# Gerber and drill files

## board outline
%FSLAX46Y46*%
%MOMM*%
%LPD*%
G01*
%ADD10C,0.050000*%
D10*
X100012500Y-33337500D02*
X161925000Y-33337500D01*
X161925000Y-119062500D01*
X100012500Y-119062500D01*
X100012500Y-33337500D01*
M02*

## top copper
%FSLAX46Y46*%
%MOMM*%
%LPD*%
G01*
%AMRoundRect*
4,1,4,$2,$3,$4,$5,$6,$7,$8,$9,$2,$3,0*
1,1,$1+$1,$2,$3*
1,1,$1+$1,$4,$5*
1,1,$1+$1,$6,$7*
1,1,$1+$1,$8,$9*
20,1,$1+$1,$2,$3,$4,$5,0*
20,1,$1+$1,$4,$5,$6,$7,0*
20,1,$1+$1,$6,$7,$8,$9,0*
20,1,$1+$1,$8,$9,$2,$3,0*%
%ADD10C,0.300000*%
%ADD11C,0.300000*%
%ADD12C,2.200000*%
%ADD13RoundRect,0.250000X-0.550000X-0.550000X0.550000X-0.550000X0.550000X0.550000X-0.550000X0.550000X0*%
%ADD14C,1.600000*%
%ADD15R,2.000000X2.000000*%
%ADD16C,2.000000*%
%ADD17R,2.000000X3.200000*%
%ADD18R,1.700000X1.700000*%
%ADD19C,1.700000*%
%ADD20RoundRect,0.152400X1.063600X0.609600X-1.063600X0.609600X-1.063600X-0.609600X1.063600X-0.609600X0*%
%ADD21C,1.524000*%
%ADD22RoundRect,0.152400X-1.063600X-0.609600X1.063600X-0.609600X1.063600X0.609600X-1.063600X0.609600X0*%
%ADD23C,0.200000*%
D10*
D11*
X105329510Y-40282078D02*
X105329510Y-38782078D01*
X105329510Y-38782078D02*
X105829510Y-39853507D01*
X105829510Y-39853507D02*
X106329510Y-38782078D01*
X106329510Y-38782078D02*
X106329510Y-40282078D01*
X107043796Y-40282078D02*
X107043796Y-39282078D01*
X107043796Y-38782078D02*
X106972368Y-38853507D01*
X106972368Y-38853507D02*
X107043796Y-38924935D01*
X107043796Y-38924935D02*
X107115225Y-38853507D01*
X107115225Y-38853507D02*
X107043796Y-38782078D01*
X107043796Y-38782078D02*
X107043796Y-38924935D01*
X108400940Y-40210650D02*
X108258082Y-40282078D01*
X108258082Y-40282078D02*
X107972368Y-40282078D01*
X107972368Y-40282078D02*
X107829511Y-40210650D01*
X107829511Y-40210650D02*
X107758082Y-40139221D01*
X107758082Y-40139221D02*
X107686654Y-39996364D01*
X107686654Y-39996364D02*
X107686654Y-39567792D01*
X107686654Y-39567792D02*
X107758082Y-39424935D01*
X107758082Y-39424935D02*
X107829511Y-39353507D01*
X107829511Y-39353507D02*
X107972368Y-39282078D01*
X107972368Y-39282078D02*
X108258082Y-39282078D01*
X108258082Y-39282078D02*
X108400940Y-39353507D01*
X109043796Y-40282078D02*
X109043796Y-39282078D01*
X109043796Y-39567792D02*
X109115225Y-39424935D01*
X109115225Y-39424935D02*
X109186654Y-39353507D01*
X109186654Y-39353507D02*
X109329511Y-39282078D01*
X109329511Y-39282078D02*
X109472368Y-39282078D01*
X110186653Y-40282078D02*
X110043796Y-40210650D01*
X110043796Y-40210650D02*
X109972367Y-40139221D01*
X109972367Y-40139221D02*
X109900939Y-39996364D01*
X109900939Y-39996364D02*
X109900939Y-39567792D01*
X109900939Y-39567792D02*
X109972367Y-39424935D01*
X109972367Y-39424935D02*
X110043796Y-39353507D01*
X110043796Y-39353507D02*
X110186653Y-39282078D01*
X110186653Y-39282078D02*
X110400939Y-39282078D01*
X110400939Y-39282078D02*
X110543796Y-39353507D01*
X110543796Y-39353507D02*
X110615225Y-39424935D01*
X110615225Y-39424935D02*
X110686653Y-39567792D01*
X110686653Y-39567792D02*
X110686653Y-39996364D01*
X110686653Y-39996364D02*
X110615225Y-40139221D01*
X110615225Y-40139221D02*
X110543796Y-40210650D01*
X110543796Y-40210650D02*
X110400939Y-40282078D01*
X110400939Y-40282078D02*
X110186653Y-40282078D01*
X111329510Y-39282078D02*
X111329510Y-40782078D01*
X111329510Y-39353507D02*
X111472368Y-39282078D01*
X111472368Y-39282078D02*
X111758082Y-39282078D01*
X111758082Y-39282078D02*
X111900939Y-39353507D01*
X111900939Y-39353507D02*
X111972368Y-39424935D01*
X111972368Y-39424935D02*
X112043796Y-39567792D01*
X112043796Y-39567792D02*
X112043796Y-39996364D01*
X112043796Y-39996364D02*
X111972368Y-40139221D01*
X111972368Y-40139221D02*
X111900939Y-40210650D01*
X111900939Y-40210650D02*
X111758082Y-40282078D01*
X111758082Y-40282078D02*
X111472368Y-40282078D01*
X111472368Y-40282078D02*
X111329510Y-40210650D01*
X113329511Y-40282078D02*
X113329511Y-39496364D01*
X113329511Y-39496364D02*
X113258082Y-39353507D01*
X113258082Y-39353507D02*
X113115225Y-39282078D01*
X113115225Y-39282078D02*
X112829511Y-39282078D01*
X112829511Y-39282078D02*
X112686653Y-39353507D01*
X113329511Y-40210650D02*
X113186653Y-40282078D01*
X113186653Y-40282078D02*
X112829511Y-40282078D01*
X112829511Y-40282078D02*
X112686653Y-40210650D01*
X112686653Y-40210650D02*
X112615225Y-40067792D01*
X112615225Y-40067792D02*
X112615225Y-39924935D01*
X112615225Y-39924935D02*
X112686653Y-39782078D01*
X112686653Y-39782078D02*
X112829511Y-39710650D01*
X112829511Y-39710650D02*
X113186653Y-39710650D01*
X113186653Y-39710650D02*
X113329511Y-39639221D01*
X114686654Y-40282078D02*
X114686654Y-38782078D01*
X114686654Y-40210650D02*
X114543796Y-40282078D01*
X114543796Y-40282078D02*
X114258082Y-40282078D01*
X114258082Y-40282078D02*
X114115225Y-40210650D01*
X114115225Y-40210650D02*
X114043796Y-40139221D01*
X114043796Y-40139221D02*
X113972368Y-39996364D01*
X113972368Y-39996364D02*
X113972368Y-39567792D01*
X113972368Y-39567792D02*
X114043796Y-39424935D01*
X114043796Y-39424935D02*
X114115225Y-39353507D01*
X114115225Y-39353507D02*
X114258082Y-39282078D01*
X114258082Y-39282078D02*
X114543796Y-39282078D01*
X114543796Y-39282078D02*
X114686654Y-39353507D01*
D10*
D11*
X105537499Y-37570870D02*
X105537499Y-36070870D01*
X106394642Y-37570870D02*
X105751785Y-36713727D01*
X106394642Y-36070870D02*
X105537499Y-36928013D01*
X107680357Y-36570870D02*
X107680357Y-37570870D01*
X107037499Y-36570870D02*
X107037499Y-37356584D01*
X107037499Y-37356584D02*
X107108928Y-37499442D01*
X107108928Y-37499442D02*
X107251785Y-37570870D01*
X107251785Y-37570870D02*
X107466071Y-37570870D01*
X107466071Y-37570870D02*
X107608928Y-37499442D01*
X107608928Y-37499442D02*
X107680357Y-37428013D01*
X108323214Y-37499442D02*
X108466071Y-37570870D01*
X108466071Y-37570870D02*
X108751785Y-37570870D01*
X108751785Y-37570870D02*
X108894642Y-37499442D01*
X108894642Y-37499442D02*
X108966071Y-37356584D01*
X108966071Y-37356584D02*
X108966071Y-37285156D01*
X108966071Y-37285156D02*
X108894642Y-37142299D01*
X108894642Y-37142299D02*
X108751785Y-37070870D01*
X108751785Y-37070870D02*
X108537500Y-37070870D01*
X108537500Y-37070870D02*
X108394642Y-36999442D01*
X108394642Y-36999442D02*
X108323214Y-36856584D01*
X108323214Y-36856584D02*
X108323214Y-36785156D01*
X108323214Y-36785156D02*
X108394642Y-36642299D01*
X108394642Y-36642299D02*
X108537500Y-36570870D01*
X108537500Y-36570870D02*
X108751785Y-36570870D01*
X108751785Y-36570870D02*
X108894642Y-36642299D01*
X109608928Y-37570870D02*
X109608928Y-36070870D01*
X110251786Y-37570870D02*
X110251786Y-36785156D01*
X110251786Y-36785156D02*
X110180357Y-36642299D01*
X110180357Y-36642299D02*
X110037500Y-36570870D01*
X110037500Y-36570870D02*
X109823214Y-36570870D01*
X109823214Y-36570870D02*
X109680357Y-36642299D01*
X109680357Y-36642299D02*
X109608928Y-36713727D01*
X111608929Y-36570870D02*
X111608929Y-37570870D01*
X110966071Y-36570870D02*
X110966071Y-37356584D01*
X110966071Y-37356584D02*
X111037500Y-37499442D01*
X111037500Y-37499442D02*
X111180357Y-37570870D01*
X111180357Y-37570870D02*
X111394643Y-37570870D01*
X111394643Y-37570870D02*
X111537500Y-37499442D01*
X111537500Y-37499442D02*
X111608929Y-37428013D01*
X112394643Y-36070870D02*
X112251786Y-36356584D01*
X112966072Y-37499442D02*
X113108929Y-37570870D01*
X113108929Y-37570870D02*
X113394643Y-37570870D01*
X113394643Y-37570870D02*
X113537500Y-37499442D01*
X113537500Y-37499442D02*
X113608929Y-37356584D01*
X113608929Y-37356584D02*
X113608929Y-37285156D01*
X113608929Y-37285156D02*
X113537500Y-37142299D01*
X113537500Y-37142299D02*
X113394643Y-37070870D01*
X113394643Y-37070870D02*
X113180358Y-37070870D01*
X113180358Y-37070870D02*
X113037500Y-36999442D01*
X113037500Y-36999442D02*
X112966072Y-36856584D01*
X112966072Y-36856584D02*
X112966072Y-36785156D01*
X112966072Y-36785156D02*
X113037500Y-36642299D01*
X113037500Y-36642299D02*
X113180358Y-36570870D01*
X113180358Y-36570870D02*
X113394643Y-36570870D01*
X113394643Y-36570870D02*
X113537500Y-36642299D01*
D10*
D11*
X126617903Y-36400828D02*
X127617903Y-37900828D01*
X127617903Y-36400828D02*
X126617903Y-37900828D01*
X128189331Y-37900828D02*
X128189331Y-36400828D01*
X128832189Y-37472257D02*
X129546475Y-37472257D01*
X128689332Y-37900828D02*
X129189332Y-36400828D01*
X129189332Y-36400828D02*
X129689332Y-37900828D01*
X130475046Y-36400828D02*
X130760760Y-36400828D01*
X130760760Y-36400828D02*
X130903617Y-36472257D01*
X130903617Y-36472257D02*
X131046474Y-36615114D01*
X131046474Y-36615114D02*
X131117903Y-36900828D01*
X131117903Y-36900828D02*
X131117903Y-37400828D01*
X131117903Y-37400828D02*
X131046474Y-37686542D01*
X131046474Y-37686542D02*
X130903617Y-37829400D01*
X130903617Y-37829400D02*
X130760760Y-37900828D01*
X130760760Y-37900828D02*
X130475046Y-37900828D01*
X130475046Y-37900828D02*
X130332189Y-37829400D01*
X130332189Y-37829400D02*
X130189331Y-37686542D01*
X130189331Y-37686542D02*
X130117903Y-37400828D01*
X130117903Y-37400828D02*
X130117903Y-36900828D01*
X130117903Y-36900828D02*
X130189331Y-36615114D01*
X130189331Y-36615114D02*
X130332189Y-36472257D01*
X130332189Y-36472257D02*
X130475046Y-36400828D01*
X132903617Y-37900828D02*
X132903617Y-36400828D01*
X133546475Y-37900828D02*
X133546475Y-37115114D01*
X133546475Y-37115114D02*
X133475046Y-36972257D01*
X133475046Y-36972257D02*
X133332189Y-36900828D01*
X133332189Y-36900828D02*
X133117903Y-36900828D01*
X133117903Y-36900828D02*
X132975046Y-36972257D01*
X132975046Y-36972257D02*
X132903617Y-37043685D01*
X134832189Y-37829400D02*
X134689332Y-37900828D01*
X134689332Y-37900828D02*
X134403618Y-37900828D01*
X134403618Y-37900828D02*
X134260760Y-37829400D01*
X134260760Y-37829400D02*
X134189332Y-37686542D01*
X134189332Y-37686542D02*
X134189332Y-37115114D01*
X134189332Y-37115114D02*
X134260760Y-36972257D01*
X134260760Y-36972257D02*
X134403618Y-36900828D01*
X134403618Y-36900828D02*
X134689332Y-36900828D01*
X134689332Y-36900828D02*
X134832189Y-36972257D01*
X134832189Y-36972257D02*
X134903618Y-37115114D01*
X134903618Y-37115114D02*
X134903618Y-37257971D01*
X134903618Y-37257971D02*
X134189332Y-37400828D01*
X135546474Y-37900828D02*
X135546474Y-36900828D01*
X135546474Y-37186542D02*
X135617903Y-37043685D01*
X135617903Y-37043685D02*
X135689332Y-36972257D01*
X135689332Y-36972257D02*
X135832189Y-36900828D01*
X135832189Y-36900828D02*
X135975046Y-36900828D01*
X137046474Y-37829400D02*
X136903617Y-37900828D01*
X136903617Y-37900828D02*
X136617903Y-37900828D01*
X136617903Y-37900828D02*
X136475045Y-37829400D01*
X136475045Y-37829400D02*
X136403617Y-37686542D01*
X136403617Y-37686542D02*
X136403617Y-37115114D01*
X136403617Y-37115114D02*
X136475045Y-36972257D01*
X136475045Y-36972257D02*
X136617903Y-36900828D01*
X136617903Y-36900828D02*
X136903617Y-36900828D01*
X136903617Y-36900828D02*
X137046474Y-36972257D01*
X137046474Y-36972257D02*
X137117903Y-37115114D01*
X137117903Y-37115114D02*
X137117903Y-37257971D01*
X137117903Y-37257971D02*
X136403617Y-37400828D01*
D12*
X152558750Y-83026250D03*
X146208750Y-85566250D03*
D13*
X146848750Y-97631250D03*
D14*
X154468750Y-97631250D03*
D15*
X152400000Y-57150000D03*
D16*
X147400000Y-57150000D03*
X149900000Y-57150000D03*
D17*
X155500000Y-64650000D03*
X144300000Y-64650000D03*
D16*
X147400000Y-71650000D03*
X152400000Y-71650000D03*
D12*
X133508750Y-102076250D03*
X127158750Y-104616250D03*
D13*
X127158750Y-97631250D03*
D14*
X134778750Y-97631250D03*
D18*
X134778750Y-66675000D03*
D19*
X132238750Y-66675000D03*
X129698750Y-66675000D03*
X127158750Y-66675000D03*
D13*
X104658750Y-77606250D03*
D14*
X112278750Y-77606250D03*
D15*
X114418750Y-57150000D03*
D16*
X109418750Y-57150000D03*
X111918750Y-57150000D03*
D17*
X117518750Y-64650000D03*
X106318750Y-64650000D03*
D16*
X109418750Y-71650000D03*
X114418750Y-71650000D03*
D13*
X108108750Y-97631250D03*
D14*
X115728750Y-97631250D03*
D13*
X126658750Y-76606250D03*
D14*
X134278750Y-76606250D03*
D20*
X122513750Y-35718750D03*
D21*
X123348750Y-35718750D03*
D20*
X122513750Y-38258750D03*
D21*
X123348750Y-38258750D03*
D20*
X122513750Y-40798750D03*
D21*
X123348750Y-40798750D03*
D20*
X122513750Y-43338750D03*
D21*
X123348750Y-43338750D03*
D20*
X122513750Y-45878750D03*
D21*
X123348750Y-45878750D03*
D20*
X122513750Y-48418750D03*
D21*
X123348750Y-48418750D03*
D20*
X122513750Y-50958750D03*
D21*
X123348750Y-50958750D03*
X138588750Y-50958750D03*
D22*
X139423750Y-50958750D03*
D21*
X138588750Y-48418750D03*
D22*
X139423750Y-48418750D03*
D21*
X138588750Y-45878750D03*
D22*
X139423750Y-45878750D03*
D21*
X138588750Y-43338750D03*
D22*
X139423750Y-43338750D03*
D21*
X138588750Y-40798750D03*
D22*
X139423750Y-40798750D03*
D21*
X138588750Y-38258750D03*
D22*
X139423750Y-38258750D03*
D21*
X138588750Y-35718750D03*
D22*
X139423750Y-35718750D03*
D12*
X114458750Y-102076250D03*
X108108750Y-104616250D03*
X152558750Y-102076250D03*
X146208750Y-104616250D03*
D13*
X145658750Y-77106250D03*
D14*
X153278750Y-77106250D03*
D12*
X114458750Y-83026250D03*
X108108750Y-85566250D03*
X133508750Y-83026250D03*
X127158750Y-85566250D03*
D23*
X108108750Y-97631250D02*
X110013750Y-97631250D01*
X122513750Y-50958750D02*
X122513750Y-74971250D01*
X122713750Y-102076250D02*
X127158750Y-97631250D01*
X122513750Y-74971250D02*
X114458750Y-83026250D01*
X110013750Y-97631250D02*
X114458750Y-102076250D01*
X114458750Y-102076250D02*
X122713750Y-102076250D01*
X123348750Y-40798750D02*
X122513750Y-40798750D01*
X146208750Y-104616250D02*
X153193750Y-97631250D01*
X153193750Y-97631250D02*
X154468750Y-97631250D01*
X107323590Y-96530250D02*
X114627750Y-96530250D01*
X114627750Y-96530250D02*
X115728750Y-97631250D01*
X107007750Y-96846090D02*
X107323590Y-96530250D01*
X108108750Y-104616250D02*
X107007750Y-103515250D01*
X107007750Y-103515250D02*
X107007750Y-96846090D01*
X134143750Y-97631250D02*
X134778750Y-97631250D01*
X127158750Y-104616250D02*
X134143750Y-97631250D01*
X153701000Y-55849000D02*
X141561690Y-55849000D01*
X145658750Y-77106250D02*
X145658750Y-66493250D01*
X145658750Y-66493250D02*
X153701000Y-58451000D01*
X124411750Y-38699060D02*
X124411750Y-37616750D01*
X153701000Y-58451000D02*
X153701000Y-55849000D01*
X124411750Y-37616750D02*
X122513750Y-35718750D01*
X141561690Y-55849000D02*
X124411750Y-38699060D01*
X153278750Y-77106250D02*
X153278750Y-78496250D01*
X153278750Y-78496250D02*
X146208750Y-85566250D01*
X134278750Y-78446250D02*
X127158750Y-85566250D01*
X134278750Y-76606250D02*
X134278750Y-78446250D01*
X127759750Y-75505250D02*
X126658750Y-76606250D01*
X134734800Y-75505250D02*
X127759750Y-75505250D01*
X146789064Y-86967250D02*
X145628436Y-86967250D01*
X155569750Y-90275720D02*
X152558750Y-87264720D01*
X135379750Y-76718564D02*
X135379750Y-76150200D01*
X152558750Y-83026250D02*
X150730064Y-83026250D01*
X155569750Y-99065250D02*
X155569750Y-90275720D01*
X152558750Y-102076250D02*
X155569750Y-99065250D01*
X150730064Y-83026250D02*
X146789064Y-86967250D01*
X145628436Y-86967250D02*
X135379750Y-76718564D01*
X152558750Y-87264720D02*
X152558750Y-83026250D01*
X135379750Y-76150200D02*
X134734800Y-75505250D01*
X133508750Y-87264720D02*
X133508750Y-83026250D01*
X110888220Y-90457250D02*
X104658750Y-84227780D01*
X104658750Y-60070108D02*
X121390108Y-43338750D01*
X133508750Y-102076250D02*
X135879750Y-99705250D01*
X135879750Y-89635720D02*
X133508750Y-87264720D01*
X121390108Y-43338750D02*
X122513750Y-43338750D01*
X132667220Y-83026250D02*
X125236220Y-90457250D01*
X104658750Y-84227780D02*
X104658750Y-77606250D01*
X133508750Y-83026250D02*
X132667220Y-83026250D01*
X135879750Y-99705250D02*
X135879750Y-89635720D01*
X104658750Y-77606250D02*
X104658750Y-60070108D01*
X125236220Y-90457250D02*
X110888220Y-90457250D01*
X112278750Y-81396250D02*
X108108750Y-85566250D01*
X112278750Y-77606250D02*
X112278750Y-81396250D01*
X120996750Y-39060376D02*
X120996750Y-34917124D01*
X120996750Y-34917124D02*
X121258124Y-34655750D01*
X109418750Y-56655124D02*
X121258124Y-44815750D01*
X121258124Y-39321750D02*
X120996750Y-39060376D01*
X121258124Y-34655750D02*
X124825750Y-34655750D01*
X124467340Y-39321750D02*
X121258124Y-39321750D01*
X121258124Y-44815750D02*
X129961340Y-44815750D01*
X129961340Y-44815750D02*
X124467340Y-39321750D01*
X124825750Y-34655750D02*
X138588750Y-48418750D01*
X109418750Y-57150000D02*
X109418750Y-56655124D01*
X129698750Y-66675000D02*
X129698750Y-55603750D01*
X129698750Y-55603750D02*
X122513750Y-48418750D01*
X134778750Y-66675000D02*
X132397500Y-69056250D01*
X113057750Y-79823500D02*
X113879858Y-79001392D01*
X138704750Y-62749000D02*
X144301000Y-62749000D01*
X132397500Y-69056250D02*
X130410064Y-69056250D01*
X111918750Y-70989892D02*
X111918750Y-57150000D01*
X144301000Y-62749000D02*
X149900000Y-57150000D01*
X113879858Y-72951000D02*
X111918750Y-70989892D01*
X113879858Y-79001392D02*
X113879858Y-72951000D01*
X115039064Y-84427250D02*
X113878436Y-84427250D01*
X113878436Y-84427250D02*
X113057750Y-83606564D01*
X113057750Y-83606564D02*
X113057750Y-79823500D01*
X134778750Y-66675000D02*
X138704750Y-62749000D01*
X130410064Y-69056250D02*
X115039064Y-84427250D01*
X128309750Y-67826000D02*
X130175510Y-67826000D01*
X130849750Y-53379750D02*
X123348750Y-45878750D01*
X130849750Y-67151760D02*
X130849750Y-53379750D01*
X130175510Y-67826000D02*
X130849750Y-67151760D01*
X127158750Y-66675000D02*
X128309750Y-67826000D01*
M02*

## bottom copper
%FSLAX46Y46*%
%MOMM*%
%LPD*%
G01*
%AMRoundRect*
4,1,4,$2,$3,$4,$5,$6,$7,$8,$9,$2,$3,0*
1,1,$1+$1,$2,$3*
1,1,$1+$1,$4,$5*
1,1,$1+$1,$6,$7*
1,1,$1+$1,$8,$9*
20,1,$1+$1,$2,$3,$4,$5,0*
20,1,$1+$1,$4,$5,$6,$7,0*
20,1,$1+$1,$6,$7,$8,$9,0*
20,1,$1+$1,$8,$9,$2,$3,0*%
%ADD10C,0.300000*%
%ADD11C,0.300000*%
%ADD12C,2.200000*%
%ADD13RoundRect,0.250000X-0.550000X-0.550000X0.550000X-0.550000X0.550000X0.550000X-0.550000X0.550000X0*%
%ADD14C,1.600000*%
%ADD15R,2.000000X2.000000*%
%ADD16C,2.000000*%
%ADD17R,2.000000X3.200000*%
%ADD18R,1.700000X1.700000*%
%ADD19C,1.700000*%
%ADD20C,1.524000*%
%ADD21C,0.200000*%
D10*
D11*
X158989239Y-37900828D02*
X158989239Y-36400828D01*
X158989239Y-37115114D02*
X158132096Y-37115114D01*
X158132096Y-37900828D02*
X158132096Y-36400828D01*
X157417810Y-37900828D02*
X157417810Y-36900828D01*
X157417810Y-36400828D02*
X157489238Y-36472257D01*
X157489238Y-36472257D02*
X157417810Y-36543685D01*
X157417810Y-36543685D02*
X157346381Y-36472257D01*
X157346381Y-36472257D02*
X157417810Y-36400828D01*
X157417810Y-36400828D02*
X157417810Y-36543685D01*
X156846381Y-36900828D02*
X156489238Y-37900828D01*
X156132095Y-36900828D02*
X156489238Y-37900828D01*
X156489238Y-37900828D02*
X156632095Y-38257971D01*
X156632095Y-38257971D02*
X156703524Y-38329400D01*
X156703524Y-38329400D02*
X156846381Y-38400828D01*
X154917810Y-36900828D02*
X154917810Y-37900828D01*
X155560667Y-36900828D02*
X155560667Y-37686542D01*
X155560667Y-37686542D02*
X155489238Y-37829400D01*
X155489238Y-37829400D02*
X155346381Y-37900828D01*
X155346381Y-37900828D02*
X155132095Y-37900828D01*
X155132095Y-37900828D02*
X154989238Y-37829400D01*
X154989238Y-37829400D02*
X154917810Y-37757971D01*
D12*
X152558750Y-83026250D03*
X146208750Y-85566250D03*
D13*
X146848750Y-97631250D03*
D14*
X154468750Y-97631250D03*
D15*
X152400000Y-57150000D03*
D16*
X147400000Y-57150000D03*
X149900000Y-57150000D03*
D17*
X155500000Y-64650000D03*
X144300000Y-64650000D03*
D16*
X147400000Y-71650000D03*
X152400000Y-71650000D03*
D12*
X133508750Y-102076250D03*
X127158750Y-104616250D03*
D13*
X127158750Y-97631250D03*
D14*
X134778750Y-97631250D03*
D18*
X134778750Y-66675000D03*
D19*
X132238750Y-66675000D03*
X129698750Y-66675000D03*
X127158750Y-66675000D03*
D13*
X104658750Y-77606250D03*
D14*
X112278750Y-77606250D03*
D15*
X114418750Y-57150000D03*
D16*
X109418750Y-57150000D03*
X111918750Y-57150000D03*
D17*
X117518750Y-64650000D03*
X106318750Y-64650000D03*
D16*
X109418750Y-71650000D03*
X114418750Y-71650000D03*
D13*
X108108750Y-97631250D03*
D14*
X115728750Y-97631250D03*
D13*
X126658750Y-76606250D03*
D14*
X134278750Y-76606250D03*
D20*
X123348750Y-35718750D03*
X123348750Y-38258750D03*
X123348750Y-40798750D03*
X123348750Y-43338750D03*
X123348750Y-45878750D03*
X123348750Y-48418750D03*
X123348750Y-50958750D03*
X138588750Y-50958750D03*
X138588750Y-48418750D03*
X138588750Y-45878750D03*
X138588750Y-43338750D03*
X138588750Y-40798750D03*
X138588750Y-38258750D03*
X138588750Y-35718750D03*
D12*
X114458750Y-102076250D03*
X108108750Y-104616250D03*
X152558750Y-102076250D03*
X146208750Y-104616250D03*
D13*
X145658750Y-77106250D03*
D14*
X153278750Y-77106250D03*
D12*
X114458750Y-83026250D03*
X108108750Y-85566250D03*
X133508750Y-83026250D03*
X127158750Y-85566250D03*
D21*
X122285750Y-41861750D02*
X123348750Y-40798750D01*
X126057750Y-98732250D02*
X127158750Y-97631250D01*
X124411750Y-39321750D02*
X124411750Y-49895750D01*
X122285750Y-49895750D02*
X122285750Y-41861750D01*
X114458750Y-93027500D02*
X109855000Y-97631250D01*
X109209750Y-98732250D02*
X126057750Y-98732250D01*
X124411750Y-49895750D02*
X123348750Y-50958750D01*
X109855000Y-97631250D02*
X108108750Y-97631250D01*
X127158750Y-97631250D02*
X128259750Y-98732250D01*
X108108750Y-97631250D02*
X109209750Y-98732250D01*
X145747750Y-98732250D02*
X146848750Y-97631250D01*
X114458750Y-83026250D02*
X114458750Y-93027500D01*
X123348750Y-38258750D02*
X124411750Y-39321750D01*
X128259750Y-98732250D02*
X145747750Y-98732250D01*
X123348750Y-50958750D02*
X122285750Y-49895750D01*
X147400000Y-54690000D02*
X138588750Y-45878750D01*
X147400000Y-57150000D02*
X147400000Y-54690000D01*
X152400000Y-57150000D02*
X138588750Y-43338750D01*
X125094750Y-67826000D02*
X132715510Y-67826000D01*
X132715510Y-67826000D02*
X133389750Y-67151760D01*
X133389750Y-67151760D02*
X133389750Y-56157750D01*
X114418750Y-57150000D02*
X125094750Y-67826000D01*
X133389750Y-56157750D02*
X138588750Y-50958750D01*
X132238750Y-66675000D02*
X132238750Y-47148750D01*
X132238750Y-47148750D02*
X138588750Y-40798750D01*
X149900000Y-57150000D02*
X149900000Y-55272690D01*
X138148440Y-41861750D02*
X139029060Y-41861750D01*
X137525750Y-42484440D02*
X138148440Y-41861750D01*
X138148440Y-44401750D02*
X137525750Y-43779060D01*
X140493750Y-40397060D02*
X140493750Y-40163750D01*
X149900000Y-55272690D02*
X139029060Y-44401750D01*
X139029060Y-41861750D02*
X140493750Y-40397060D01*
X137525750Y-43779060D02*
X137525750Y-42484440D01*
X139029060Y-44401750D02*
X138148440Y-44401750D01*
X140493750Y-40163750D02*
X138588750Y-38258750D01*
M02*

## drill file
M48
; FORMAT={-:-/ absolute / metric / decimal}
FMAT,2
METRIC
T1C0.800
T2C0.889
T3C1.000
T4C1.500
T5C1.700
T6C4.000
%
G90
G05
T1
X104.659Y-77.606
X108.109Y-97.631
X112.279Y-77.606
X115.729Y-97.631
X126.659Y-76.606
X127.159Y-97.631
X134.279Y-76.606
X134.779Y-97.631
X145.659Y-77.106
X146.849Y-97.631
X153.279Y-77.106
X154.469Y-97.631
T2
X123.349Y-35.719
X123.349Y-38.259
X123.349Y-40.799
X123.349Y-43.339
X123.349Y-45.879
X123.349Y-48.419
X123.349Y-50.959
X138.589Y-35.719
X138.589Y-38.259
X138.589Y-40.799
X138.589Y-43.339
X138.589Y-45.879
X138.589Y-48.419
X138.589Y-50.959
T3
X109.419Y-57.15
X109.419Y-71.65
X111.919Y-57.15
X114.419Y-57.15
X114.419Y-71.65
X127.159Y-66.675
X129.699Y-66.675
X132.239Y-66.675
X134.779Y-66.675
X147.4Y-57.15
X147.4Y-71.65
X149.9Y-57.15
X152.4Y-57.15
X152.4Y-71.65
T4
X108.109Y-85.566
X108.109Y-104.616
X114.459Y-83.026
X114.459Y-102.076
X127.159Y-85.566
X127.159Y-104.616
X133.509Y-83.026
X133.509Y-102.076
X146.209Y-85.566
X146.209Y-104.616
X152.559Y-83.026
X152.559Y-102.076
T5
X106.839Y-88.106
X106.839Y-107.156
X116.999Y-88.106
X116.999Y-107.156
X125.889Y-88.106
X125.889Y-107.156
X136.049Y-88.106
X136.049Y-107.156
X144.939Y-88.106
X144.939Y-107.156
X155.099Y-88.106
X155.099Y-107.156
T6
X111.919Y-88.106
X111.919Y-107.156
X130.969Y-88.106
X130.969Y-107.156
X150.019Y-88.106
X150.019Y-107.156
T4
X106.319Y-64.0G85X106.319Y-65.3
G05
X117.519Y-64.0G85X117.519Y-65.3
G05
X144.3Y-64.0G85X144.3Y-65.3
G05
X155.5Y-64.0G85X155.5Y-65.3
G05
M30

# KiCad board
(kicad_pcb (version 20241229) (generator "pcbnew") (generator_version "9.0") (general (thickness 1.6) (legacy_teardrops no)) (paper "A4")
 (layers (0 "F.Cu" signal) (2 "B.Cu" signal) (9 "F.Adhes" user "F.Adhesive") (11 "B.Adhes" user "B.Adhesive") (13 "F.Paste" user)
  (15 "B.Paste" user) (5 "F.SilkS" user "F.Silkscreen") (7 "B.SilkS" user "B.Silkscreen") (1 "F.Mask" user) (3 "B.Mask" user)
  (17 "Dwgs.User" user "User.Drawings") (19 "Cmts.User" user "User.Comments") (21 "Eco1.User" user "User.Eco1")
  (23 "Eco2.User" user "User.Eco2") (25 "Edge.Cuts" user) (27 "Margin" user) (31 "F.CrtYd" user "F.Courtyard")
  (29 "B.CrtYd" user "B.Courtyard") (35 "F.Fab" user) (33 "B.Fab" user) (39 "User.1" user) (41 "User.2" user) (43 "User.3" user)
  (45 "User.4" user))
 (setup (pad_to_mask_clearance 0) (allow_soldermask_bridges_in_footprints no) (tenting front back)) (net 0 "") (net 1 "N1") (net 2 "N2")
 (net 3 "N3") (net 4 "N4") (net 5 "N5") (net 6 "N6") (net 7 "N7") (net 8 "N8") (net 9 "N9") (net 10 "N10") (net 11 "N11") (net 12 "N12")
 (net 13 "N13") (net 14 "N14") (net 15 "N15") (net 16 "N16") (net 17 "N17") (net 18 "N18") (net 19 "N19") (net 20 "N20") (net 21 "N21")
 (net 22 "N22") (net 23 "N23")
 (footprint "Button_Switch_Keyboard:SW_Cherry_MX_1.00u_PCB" (layer "F.Cu") (at 152.55875 83.02625)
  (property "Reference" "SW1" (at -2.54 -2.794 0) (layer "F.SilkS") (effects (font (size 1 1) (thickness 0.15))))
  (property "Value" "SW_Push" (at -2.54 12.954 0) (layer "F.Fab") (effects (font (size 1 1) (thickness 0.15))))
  (pad "" np_thru_hole circle (at -7.62 5.08) (size 1.7 1.7) (drill 1.7) (layers "*.Cu" "*.Mask"))
  (pad "" np_thru_hole circle (at -2.54 5.08) (size 4 4) (drill 4) (layers "*.Cu" "*.Mask"))
  (pad "" np_thru_hole circle (at 2.54 5.08) (size 1.7 1.7) (drill 1.7) (layers "*.Cu" "*.Mask"))
  (pad "1" thru_hole circle (at 0 0) (size 2.2 2.2) (drill 1.5) (layers "*.Cu" "*.Mask") (remove_unused_layers no) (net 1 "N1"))
  (pad "2" thru_hole circle (at -6.35 2.54) (size 2.2 2.2) (drill 1.5) (layers "*.Cu" "*.Mask") (remove_unused_layers no) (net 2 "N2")))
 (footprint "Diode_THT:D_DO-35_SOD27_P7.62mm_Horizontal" (layer "F.Cu") (at 146.84875 97.63125)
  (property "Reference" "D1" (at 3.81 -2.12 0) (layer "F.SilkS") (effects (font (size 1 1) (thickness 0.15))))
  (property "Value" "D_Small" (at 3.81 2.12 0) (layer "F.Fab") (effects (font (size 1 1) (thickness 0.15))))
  (pad "1" thru_hole roundrect (at 0 0) (size 1.6 1.6) (drill 0.8) (layers "*.Cu" "*.Mask") (remove_unused_layers no)
   (roundrect_rratio 0.15625) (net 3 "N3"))
  (pad "2" thru_hole circle (at 7.62 0) (size 1.6 1.6) (drill 0.8) (layers "*.Cu" "*.Mask") (remove_unused_layers no) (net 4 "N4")))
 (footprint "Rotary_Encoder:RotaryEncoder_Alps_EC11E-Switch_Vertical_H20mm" (layer "F.Cu") (at 152.4 57.15 -90)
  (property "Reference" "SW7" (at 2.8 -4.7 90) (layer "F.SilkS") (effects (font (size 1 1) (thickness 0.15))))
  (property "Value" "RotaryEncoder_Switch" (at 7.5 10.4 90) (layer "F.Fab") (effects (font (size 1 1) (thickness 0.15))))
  (pad "A" thru_hole rect (at 0 0 270) (size 2 2) (drill 1) (layers "*.Cu" "*.Mask") (remove_unused_layers no) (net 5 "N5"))
  (pad "B" thru_hole circle (at 0 5 270) (size 2 2) (drill 1) (layers "*.Cu" "*.Mask") (remove_unused_layers no) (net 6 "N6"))
  (pad "C" thru_hole circle (at 0 2.5 270) (size 2 2) (drill 1) (layers "*.Cu" "*.Mask") (remove_unused_layers no) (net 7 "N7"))
  (pad "MP" thru_hole rect (at 7.5 -3.1 270) (size 3.2 2) (drill oval 2.8 1.5) (layers "*.Cu" "*.Mask") (remove_unused_layers no))
  (pad "MP" thru_hole rect (at 7.5 8.1 270) (size 3.2 2) (drill oval 2.8 1.5) (layers "*.Cu" "*.Mask") (remove_unused_layers no))
  (pad "S1" thru_hole circle (at 14.5 5 270) (size 2 2) (drill 1) (layers "*.Cu" "*.Mask") (remove_unused_layers no) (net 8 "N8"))
  (pad "S2" thru_hole circle (at 14.5 0 270) (size 2 2) (drill 1) (layers "*.Cu" "*.Mask") (remove_unused_layers no) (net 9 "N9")))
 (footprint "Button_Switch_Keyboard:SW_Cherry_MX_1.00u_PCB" (layer "F.Cu") (at 133.50875 102.07625)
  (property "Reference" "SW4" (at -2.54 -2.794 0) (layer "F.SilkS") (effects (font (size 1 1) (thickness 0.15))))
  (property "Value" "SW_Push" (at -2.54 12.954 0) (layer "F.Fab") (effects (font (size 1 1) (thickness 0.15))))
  (pad "" np_thru_hole circle (at -7.62 5.08) (size 1.7 1.7) (drill 1.7) (layers "*.Cu" "*.Mask"))
  (pad "" np_thru_hole circle (at -2.54 5.08) (size 4 4) (drill 4) (layers "*.Cu" "*.Mask"))
  (pad "" np_thru_hole circle (at 2.54 5.08) (size 1.7 1.7) (drill 1.7) (layers "*.Cu" "*.Mask"))
  (pad "1" thru_hole circle (at 0 0) (size 2.2 2.2) (drill 1.5) (layers "*.Cu" "*.Mask") (remove_unused_layers no) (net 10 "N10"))
  (pad "2" thru_hole circle (at -6.35 2.54) (size 2.2 2.2) (drill 1.5) (layers "*.Cu" "*.Mask") (remove_unused_layers no) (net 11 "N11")))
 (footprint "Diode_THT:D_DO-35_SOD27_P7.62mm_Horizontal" (layer "F.Cu") (at 127.15875 97.63125)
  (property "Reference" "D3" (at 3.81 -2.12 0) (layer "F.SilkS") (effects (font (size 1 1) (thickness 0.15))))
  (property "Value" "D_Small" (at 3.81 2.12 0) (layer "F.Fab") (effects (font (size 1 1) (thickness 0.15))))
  (pad "1" thru_hole roundrect (at 0 0) (size 1.6 1.6) (drill 0.8) (layers "*.Cu" "*.Mask") (remove_unused_layers no)
   (roundrect_rratio 0.15625) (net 3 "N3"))
  (pad "2" thru_hole circle (at 7.62 0) (size 1.6 1.6) (drill 0.8) (layers "*.Cu" "*.Mask") (remove_unused_layers no) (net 11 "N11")))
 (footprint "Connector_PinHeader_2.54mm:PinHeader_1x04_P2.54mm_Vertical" (layer "F.Cu") (at 134.77875 66.675 -90)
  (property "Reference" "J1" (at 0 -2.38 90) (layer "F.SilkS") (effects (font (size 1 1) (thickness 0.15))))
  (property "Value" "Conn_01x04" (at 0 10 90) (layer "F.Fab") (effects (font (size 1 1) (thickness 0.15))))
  (pad "1" thru_hole rect (at 0 0 270) (size 1.7 1.7) (drill 1) (layers "*.Cu" "*.Mask") (remove_unused_layers no) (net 7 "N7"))
  (pad "2" thru_hole circle (at 0 2.54 270) (size 1.7 1.7) (drill 1) (layers "*.Cu" "*.Mask") (remove_unused_layers no) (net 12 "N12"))
  (pad "3" thru_hole circle (at 0 5.08 270) (size 1.7 1.7) (drill 1) (layers "*.Cu" "*.Mask") (remove_unused_layers no) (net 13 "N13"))
  (pad "4" thru_hole circle (at 0 7.62 270) (size 1.7 1.7) (drill 1) (layers "*.Cu" "*.Mask") (remove_unused_layers no) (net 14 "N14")))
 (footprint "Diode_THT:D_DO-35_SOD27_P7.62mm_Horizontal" (layer "F.Cu") (at 104.65875 77.60625)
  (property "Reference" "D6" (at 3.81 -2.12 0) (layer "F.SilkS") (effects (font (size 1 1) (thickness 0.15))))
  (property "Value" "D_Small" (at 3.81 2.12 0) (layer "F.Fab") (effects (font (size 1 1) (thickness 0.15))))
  (pad "1" thru_hole roundrect (at 0 0) (size 1.6 1.6) (drill 0.8) (layers "*.Cu" "*.Mask") (remove_unused_layers no)
   (roundrect_rratio 0.15625) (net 10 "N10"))
  (pad "2" thru_hole circle (at 7.62 0) (size 1.6 1.6) (drill 0.8) (layers "*.Cu" "*.Mask") (remove_unused_layers no) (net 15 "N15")))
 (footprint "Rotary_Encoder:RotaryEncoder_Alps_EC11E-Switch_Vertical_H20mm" (layer "F.Cu") (at 114.41875 57.15 -90)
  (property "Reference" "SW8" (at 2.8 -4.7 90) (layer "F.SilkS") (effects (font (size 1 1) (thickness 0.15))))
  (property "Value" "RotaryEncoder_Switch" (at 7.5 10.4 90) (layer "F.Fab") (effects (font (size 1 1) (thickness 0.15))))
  (pad "A" thru_hole rect (at 0 0 270) (size 2 2) (drill 1) (layers "*.Cu" "*.Mask") (remove_unused_layers no) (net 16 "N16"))
  (pad "B" thru_hole circle (at 0 5 270) (size 2 2) (drill 1) (layers "*.Cu" "*.Mask") (remove_unused_layers no) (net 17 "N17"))
  (pad "C" thru_hole circle (at 0 2.5 270) (size 2 2) (drill 1) (layers "*.Cu" "*.Mask") (remove_unused_layers no) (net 7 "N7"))
  (pad "MP" thru_hole rect (at 7.5 -3.1 270) (size 3.2 2) (drill oval 2.8 1.5) (layers "*.Cu" "*.Mask") (remove_unused_layers no))
  (pad "MP" thru_hole rect (at 7.5 8.1 270) (size 3.2 2) (drill oval 2.8 1.5) (layers "*.Cu" "*.Mask") (remove_unused_layers no))
  (pad "S1" thru_hole circle (at 14.5 5 270) (size 2 2) (drill 1) (layers "*.Cu" "*.Mask") (remove_unused_layers no) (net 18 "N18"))
  (pad "S2" thru_hole circle (at 14.5 0 270) (size 2 2) (drill 1) (layers "*.Cu" "*.Mask") (remove_unused_layers no) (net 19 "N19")))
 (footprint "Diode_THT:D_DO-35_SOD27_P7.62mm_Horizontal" (layer "F.Cu") (at 108.10875 97.63125)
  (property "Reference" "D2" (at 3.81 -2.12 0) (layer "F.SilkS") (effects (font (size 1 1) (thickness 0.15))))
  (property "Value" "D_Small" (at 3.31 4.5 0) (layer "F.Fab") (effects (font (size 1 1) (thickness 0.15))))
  (pad "1" thru_hole roundrect (at 0 0) (size 1.6 1.6) (drill 0.8) (layers "*.Cu" "*.Mask") (remove_unused_layers no)
   (roundrect_rratio 0.15625) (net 3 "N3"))
  (pad "2" thru_hole circle (at 7.62 0) (size 1.6 1.6) (drill 0.8) (layers "*.Cu" "*.Mask") (remove_unused_layers no) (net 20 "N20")))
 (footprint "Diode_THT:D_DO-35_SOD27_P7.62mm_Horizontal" (layer "F.Cu") (at 126.65875 76.60625)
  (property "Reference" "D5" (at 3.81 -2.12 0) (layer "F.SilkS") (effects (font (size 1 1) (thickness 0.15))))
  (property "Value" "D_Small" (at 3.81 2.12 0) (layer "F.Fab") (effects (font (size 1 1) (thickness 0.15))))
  (pad "1" thru_hole roundrect (at 0 0) (size 1.6 1.6) (drill 0.8) (layers "*.Cu" "*.Mask") (remove_unused_layers no)
   (roundrect_rratio 0.15625) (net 1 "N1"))
  (pad "2" thru_hole circle (at 7.62 0) (size 1.6 1.6) (drill 0.8) (layers "*.Cu" "*.Mask") (remove_unused_layers no) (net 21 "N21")))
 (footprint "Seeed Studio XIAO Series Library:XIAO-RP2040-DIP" (layer "F.Cu") (at 130.96875 43.33875)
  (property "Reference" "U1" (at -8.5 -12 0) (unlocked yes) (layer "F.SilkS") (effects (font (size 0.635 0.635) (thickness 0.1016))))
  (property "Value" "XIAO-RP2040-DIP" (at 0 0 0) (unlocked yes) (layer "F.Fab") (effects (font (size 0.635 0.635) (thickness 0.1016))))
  (pad "1" smd roundrect (at -8.455 -7.62 180) (size 2.432 1.524) (layers "F.Cu" "F.Mask") (roundrect_rratio 0.1) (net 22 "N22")
   (thermal_bridge_angle 45))
  (pad "1" thru_hole circle (at -7.62 -7.62 180) (size 1.524 1.524) (drill 0.889) (layers "*.Cu" "*.Mask") (remove_unused_layers no)
   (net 22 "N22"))
  (pad "2" smd roundrect (at -8.455 -5.08 180) (size 2.432 1.524) (layers "F.Cu" "F.Mask") (roundrect_rratio 0.1) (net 3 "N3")
   (thermal_bridge_angle 45))
  (pad "2" thru_hole circle (at -7.62 -5.08 180) (size 1.524 1.524) (drill 0.889) (layers "*.Cu" "*.Mask") (remove_unused_layers no)
   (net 3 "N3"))
  (pad "3" smd roundrect (at -8.455 -2.54 180) (size 2.432 1.524) (layers "F.Cu" "F.Mask") (roundrect_rratio 0.1) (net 3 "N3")
   (thermal_bridge_angle 45))
  (pad "3" thru_hole circle (at -7.62 -2.54 180) (size 1.524 1.524) (drill 0.889) (layers "*.Cu" "*.Mask") (remove_unused_layers no)
   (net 3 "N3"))
  (pad "4" smd roundrect (at -8.455 0 180) (size 2.432 1.524) (layers "F.Cu" "F.Mask") (roundrect_rratio 0.1) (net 10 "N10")
   (thermal_bridge_angle 45))
  (pad "4" thru_hole circle (at -7.62 0 180) (size 1.524 1.524) (drill 0.889) (layers "*.Cu" "*.Mask") (remove_unused_layers no)
   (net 10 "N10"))
  (pad "5" smd roundrect (at -8.455 2.54 180) (size 2.432 1.524) (layers "F.Cu" "F.Mask") (roundrect_rratio 0.1) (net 14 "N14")
   (thermal_bridge_angle 45))
  (pad "5" thru_hole circle (at -7.62 2.54 180) (size 1.524 1.524) (drill 0.889) (layers "*.Cu" "*.Mask") (remove_unused_layers no)
   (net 14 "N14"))
  (pad "6" smd roundrect (at -8.455 5.08 180) (size 2.432 1.524) (layers "F.Cu" "F.Mask") (roundrect_rratio 0.1) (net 13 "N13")
   (thermal_bridge_angle 45))
  (pad "6" thru_hole circle (at -7.62 5.08 180) (size 1.524 1.524) (drill 0.889) (layers "*.Cu" "*.Mask") (remove_unused_layers no)
   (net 13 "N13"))
  (pad "7" smd roundrect (at -8.455 7.62 180) (size 2.432 1.524) (layers "F.Cu" "F.Mask") (roundrect_rratio 0.1) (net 3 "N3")
   (thermal_bridge_angle 45))
  (pad "7" thru_hole circle (at -7.62 7.62 180) (size 1.524 1.524) (drill 0.889) (layers "*.Cu" "*.Mask") (remove_unused_layers no)
   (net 3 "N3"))
  (pad "8" thru_hole circle (at 7.62 7.62) (size 1.524 1.524) (drill 0.889) (layers "*.Cu" "*.Mask") (remove_unused_layers no)
   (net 16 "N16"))
  (pad "8" smd roundrect (at 8.455 7.62) (size 2.432 1.524) (layers "F.Cu" "F.Mask") (roundrect_rratio 0.1) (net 16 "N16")
   (thermal_bridge_angle 45))
  (pad "9" thru_hole circle (at 7.62 5.08) (size 1.524 1.524) (drill 0.889) (layers "*.Cu" "*.Mask") (remove_unused_layers no)
   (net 17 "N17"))
  (pad "9" smd roundrect (at 8.455 5.08) (size 2.432 1.524) (layers "F.Cu" "F.Mask") (roundrect_rratio 0.1) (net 17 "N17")
   (thermal_bridge_angle 45))
  (pad "10" thru_hole circle (at 7.62 2.54) (size 1.524 1.524) (drill 0.889) (layers "*.Cu" "*.Mask") (remove_unused_layers no) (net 6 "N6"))
  (pad "10" smd roundrect (at 8.455 2.54) (size 2.432 1.524) (layers "F.Cu" "F.Mask") (roundrect_rratio 0.1) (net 6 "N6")
   (thermal_bridge_angle 45))
  (pad "11" thru_hole circle (at 7.62 0) (size 1.524 1.524) (drill 0.889) (layers "*.Cu" "*.Mask") (remove_unused_layers no) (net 5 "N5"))
  (pad "11" smd roundrect (at 8.455 0) (size 2.432 1.524) (layers "F.Cu" "F.Mask") (roundrect_rratio 0.1) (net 5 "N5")
   (thermal_bridge_angle 45))
  (pad "12" thru_hole circle (at 7.62 -2.54) (size 1.524 1.524) (drill 0.889) (layers "*.Cu" "*.Mask") (remove_unused_layers no)
   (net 12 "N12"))
  (pad "12" smd roundrect (at 8.455 -2.54) (size 2.432 1.524) (layers "F.Cu" "F.Mask") (roundrect_rratio 0.1) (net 12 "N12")
   (thermal_bridge_angle 45))
  (pad "13" thru_hole circle (at 7.62 -5.08) (size 1.524 1.524) (drill 0.889) (layers "*.Cu" "*.Mask") (remove_unused_layers no)
   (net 7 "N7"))
  (pad "13" smd roundrect (at 8.455 -5.08) (size 2.432 1.524) (layers "F.Cu" "F.Mask") (roundrect_rratio 0.1) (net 7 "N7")
   (thermal_bridge_angle 45))
  (pad "14" thru_hole circle (at 7.62 -7.62) (size 1.524 1.524) (drill 0.889) (layers "*.Cu" "*.Mask") (remove_unused_layers no)
   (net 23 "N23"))
  (pad "14" smd roundrect (at 8.455 -7.62) (size 2.432 1.524) (layers "F.Cu" "F.Mask") (roundrect_rratio 0.1) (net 23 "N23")
   (thermal_bridge_angle 45)))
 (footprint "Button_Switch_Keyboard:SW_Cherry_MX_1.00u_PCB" (layer "F.Cu") (at 114.45875 102.07625)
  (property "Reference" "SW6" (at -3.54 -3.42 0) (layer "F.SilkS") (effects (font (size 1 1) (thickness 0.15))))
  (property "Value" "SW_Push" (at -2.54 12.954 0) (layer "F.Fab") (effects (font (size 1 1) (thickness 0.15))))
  (pad "" np_thru_hole circle (at -7.62 5.08) (size 1.7 1.7) (drill 1.7) (layers "*.Cu" "*.Mask"))
  (pad "" np_thru_hole circle (at -2.54 5.08) (size 4 4) (drill 4) (layers "*.Cu" "*.Mask"))
  (pad "" np_thru_hole circle (at 2.54 5.08) (size 1.7 1.7) (drill 1.7) (layers "*.Cu" "*.Mask"))
  (pad "1" thru_hole circle (at 0 0) (size 2.2 2.2) (drill 1.5) (layers "*.Cu" "*.Mask") (remove_unused_layers no) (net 3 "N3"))
  (pad "2" thru_hole circle (at -6.35 2.54) (size 2.2 2.2) (drill 1.5) (layers "*.Cu" "*.Mask") (remove_unused_layers no) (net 20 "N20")))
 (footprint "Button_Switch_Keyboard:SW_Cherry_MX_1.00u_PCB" (layer "F.Cu") (at 152.55875 102.07625)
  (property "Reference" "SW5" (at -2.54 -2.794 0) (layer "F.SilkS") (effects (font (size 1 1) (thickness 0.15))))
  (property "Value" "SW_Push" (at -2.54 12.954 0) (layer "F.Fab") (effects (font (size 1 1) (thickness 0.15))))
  (pad "" np_thru_hole circle (at -7.62 5.08) (size 1.7 1.7) (drill 1.7) (layers "*.Cu" "*.Mask"))
  (pad "" np_thru_hole circle (at -2.54 5.08) (size 4 4) (drill 4) (layers "*.Cu" "*.Mask"))
  (pad "" np_thru_hole circle (at 2.54 5.08) (size 1.7 1.7) (drill 1.7) (layers "*.Cu" "*.Mask"))
  (pad "1" thru_hole circle (at 0 0) (size 2.2 2.2) (drill 1.5) (layers "*.Cu" "*.Mask") (remove_unused_layers no) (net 1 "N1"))
  (pad "2" thru_hole circle (at -6.35 2.54) (size 2.2 2.2) (drill 1.5) (layers "*.Cu" "*.Mask") (remove_unused_layers no) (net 4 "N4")))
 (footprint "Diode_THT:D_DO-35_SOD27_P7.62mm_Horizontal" (layer "F.Cu") (at 145.65875 77.10625)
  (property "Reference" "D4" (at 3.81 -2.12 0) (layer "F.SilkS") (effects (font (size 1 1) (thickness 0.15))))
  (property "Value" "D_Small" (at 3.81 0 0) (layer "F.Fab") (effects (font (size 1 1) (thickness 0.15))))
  (pad "1" thru_hole roundrect (at 0 0) (size 1.6 1.6) (drill 0.8) (layers "*.Cu" "*.Mask") (remove_unused_layers no)
   (roundrect_rratio 0.15625) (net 22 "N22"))
  (pad "2" thru_hole circle (at 7.62 0) (size 1.6 1.6) (drill 0.8) (layers "*.Cu" "*.Mask") (remove_unused_layers no) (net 2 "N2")))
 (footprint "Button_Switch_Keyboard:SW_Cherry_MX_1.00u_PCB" (layer "F.Cu") (at 114.45875 83.02625)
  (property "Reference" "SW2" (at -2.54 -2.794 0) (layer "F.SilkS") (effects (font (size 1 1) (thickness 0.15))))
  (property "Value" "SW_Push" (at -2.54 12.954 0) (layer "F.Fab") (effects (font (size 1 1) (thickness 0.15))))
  (pad "" np_thru_hole circle (at -7.62 5.08) (size 1.7 1.7) (drill 1.7) (layers "*.Cu" "*.Mask"))
  (pad "" np_thru_hole circle (at -2.54 5.08) (size 4 4) (drill 4) (layers "*.Cu" "*.Mask"))
  (pad "" np_thru_hole circle (at 2.54 5.08) (size 1.7 1.7) (drill 1.7) (layers "*.Cu" "*.Mask"))
  (pad "1" thru_hole circle (at 0 0) (size 2.2 2.2) (drill 1.5) (layers "*.Cu" "*.Mask") (remove_unused_layers no) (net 3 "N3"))
  (pad "2" thru_hole circle (at -6.35 2.54) (size 2.2 2.2) (drill 1.5) (layers "*.Cu" "*.Mask") (remove_unused_layers no) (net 15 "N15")))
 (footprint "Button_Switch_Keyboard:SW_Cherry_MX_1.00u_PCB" (layer "F.Cu") (at 133.50875 83.02625)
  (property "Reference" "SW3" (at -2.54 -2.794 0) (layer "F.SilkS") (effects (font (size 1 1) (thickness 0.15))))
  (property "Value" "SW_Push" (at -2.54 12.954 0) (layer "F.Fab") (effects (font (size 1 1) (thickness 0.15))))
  (pad "" np_thru_hole circle (at -7.62 5.08) (size 1.7 1.7) (drill 1.7) (layers "*.Cu" "*.Mask"))
  (pad "" np_thru_hole circle (at -2.54 5.08) (size 4 4) (drill 4) (layers "*.Cu" "*.Mask"))
  (pad "" np_thru_hole circle (at 2.54 5.08) (size 1.7 1.7) (drill 1.7) (layers "*.Cu" "*.Mask"))
  (pad "1" thru_hole circle (at 0 0) (size 2.2 2.2) (drill 1.5) (layers "*.Cu" "*.Mask") (remove_unused_layers no) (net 10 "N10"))
  (pad "2" thru_hole circle (at -6.35 2.54) (size 2.2 2.2) (drill 1.5) (layers "*.Cu" "*.Mask") (remove_unused_layers no) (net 21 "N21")))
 (gr_rect (start 100.0125 33.3375) (end 161.925 119.0625) (stroke (width 0.05) (type default)) (fill no) (layer "Edge.Cuts"))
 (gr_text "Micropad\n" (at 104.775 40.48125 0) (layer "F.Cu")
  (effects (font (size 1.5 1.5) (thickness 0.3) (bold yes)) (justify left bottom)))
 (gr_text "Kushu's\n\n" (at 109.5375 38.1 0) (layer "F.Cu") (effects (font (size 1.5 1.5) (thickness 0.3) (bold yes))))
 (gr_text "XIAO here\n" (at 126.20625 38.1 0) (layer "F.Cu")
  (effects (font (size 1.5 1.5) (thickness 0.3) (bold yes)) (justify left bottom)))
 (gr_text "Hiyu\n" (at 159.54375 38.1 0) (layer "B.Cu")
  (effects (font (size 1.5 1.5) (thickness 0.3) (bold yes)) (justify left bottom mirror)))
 (segment (start 108.10875 97.63125) (end 110.01375 97.63125) (width 0.2) (layer "F.Cu") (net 3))
 (segment (start 122.51375 50.95875) (end 122.51375 74.97125) (width 0.2) (layer "F.Cu") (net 3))
 (segment (start 122.71375 102.07625) (end 127.15875 97.63125) (width 0.2) (layer "F.Cu") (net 3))
 (segment (start 122.51375 74.97125) (end 114.45875 83.02625) (width 0.2) (layer "F.Cu") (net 3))
 (segment (start 110.01375 97.63125) (end 114.45875 102.07625) (width 0.2) (layer "F.Cu") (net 3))
 (segment (start 114.45875 102.07625) (end 122.71375 102.07625) (width 0.2) (layer "F.Cu") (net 3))
 (segment (start 123.34875 40.79875) (end 122.51375 40.79875) (width 0.2) (layer "F.Cu") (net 3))
 (segment (start 122.28575 41.86175) (end 123.34875 40.79875) (width 0.2) (layer "B.Cu") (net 3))
 (segment (start 126.05775 98.73225) (end 127.15875 97.63125) (width 0.2) (layer "B.Cu") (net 3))
 (segment (start 124.41175 39.32175) (end 124.41175 49.89575) (width 0.2) (layer "B.Cu") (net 3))
 (segment (start 122.28575 49.89575) (end 122.28575 41.86175) (width 0.2) (layer "B.Cu") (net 3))
 (segment (start 114.45875 93.0275) (end 109.855 97.63125) (width 0.2) (layer "B.Cu") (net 3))
 (segment (start 109.20975 98.73225) (end 126.05775 98.73225) (width 0.2) (layer "B.Cu") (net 3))
 (segment (start 124.41175 49.89575) (end 123.34875 50.95875) (width 0.2) (layer "B.Cu") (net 3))
 (segment (start 109.855 97.63125) (end 108.10875 97.63125) (width 0.2) (layer "B.Cu") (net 3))
 (segment (start 127.15875 97.63125) (end 128.25975 98.73225) (width 0.2) (layer "B.Cu") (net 3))
 (segment (start 108.10875 97.63125) (end 109.20975 98.73225) (width 0.2) (layer "B.Cu") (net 3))
 (segment (start 145.74775 98.73225) (end 146.84875 97.63125) (width 0.2) (layer "B.Cu") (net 3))
 (segment (start 114.45875 83.02625) (end 114.45875 93.0275) (width 0.2) (layer "B.Cu") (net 3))
 (segment (start 123.34875 38.25875) (end 124.41175 39.32175) (width 0.2) (layer "B.Cu") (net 3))
 (segment (start 128.25975 98.73225) (end 145.74775 98.73225) (width 0.2) (layer "B.Cu") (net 3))
 (segment (start 123.34875 50.95875) (end 122.28575 49.89575) (width 0.2) (layer "B.Cu") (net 3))
 (segment (start 146.20875 104.61625) (end 153.19375 97.63125) (width 0.2) (layer "F.Cu") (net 4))
 (segment (start 153.19375 97.63125) (end 154.46875 97.63125) (width 0.2) (layer "F.Cu") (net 4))
 (segment (start 107.32359 96.53025) (end 114.62775 96.53025) (width 0.2) (layer "F.Cu") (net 20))
 (segment (start 114.62775 96.53025) (end 115.72875 97.63125) (width 0.2) (layer "F.Cu") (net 20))
 (segment (start 107.00775 96.84609) (end 107.32359 96.53025) (width 0.2) (layer "F.Cu") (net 20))
 (segment (start 108.10875 104.61625) (end 107.00775 103.51525) (width 0.2) (layer "F.Cu") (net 20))
 (segment (start 107.00775 103.51525) (end 107.00775 96.84609) (width 0.2) (layer "F.Cu") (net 20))
 (segment (start 134.14375 97.63125) (end 134.77875 97.63125) (width 0.2) (layer "F.Cu") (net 11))
 (segment (start 127.15875 104.61625) (end 134.14375 97.63125) (width 0.2) (layer "F.Cu") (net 11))
 (segment (start 153.701 55.849) (end 141.56169 55.849) (width 0.2) (layer "F.Cu") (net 22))
 (segment (start 145.65875 77.10625) (end 145.65875 66.49325) (width 0.2) (layer "F.Cu") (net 22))
 (segment (start 145.65875 66.49325) (end 153.701 58.451) (width 0.2) (layer "F.Cu") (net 22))
 (segment (start 124.41175 38.69906) (end 124.41175 37.61675) (width 0.2) (layer "F.Cu") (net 22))
 (segment (start 153.701 58.451) (end 153.701 55.849) (width 0.2) (layer "F.Cu") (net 22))
 (segment (start 124.41175 37.61675) (end 122.51375 35.71875) (width 0.2) (layer "F.Cu") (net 22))
 (segment (start 141.56169 55.849) (end 124.41175 38.69906) (width 0.2) (layer "F.Cu") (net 22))
 (segment (start 153.27875 77.10625) (end 153.27875 78.49625) (width 0.2) (layer "F.Cu") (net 2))
 (segment (start 153.27875 78.49625) (end 146.20875 85.56625) (width 0.2) (layer "F.Cu") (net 2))
 (segment (start 134.27875 78.44625) (end 127.15875 85.56625) (width 0.2) (layer "F.Cu") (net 21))
 (segment (start 134.27875 76.60625) (end 134.27875 78.44625) (width 0.2) (layer "F.Cu") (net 21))
 (segment (start 127.75975 75.50525) (end 126.65875 76.60625) (width 0.2) (layer "F.Cu") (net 1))
 (segment (start 134.7348 75.50525) (end 127.75975 75.50525) (width 0.2) (layer "F.Cu") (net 1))
 (segment (start 146.789064 86.96725) (end 145.628436 86.96725) (width 0.2) (layer "F.Cu") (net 1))
 (segment (start 155.56975 90.27572) (end 152.55875 87.26472) (width 0.2) (layer "F.Cu") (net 1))
 (segment (start 135.37975 76.718564) (end 135.37975 76.1502) (width 0.2) (layer "F.Cu") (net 1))
 (segment (start 152.55875 83.02625) (end 150.730064 83.02625) (width 0.2) (layer "F.Cu") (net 1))
 (segment (start 155.56975 99.06525) (end 155.56975 90.27572) (width 0.2) (layer "F.Cu") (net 1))
 (segment (start 152.55875 102.07625) (end 155.56975 99.06525) (width 0.2) (layer "F.Cu") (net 1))
 (segment (start 150.730064 83.02625) (end 146.789064 86.96725) (width 0.2) (layer "F.Cu") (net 1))
 (segment (start 145.628436 86.96725) (end 135.37975 76.718564) (width 0.2) (layer "F.Cu") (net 1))
 (segment (start 152.55875 87.26472) (end 152.55875 83.02625) (width 0.2) (layer "F.Cu") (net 1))
 (segment (start 135.37975 76.1502) (end 134.7348 75.50525) (width 0.2) (layer "F.Cu") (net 1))
 (segment (start 133.50875 87.26472) (end 133.50875 83.02625) (width 0.2) (layer "F.Cu") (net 10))
 (segment (start 110.88822 90.45725) (end 104.65875 84.22778) (width 0.2) (layer "F.Cu") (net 10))
 (segment (start 104.65875 60.070108) (end 121.390108 43.33875) (width 0.2) (layer "F.Cu") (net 10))
 (segment (start 133.50875 102.07625) (end 135.87975 99.70525) (width 0.2) (layer "F.Cu") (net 10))
 (segment (start 135.87975 89.63572) (end 133.50875 87.26472) (width 0.2) (layer "F.Cu") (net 10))
 (segment (start 121.390108 43.33875) (end 122.51375 43.33875) (width 0.2) (layer "F.Cu") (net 10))
 (segment (start 132.66722 83.02625) (end 125.23622 90.45725) (width 0.2) (layer "F.Cu") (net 10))
 (segment (start 104.65875 84.22778) (end 104.65875 77.60625) (width 0.2) (layer "F.Cu") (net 10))
 (segment (start 133.50875 83.02625) (end 132.66722 83.02625) (width 0.2) (layer "F.Cu") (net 10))
 (segment (start 135.87975 99.70525) (end 135.87975 89.63572) (width 0.2) (layer "F.Cu") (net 10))
 (segment (start 104.65875 77.60625) (end 104.65875 60.070108) (width 0.2) (layer "F.Cu") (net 10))
 (segment (start 125.23622 90.45725) (end 110.88822 90.45725) (width 0.2) (layer "F.Cu") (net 10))
 (segment (start 112.27875 81.39625) (end 108.10875 85.56625) (width 0.2) (layer "F.Cu") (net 15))
 (segment (start 112.27875 77.60625) (end 112.27875 81.39625) (width 0.2) (layer "F.Cu") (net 15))
 (segment (start 147.4 54.69) (end 138.58875 45.87875) (width 0.2) (layer "B.Cu") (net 6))
 (segment (start 147.4 57.15) (end 147.4 54.69) (width 0.2) (layer "B.Cu") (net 6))
 (segment (start 152.4 57.15) (end 138.58875 43.33875) (width 0.2) (layer "B.Cu") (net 5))
 (segment (start 125.09475 67.826) (end 132.71551 67.826) (width 0.2) (layer "B.Cu") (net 16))
 (segment (start 132.71551 67.826) (end 133.38975 67.15176) (width 0.2) (layer "B.Cu") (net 16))
 (segment (start 133.38975 67.15176) (end 133.38975 56.15775) (width 0.2) (layer "B.Cu") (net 16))
 (segment (start 114.41875 57.15) (end 125.09475 67.826) (width 0.2) (layer "B.Cu") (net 16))
 (segment (start 133.38975 56.15775) (end 138.58875 50.95875) (width 0.2) (layer "B.Cu") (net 16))
 (segment (start 120.99675 39.060376) (end 120.99675 34.917124) (width 0.2) (layer "F.Cu") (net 17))
 (segment (start 120.99675 34.917124) (end 121.258124 34.65575) (width 0.2) (layer "F.Cu") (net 17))
 (segment (start 109.41875 56.655124) (end 121.258124 44.81575) (width 0.2) (layer "F.Cu") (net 17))
 (segment (start 121.258124 39.32175) (end 120.99675 39.060376) (width 0.2) (layer "F.Cu") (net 17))
 (segment (start 121.258124 34.65575) (end 124.82575 34.65575) (width 0.2) (layer "F.Cu") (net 17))
 (segment (start 124.46734 39.32175) (end 121.258124 39.32175) (width 0.2) (layer "F.Cu") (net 17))
 (segment (start 121.258124 44.81575) (end 129.96134 44.81575) (width 0.2) (layer "F.Cu") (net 17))
 (segment (start 129.96134 44.81575) (end 124.46734 39.32175) (width 0.2) (layer "F.Cu") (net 17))
 (segment (start 124.82575 34.65575) (end 138.58875 48.41875) (width 0.2) (layer "F.Cu") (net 17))
 (segment (start 109.41875 57.15) (end 109.41875 56.655124) (width 0.2) (layer "F.Cu") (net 17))
 (segment (start 132.23875 66.675) (end 132.23875 47.14875) (width 0.2) (layer "B.Cu") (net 12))
 (segment (start 132.23875 47.14875) (end 138.58875 40.79875) (width 0.2) (layer "B.Cu") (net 12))
 (segment (start 129.69875 66.675) (end 129.69875 55.60375) (width 0.2) (layer "F.Cu") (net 13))
 (segment (start 129.69875 55.60375) (end 122.51375 48.41875) (width 0.2) (layer "F.Cu") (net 13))
 (segment (start 134.77875 66.675) (end 132.3975 69.05625) (width 0.2) (layer "F.Cu") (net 7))
 (segment (start 113.05775 79.8235) (end 113.879858 79.001392) (width 0.2) (layer "F.Cu") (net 7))
 (segment (start 138.70475 62.749) (end 144.301 62.749) (width 0.2) (layer "F.Cu") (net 7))
 (segment (start 132.3975 69.05625) (end 130.410064 69.05625) (width 0.2) (layer "F.Cu") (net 7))
 (segment (start 111.91875 70.989892) (end 111.91875 57.15) (width 0.2) (layer "F.Cu") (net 7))
 (segment (start 144.301 62.749) (end 149.9 57.15) (width 0.2) (layer "F.Cu") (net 7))
 (segment (start 113.879858 72.951) (end 111.91875 70.989892) (width 0.2) (layer "F.Cu") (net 7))
 (segment (start 113.879858 79.001392) (end 113.879858 72.951) (width 0.2) (layer "F.Cu") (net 7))
 (segment (start 115.039064 84.42725) (end 113.878436 84.42725) (width 0.2) (layer "F.Cu") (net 7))
 (segment (start 113.878436 84.42725) (end 113.05775 83.606564) (width 0.2) (layer "F.Cu") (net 7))
 (segment (start 113.05775 83.606564) (end 113.05775 79.8235) (width 0.2) (layer "F.Cu") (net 7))
 (segment (start 134.77875 66.675) (end 138.70475 62.749) (width 0.2) (layer "F.Cu") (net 7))
 (segment (start 130.410064 69.05625) (end 115.039064 84.42725) (width 0.2) (layer "F.Cu") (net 7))
 (segment (start 149.9 57.15) (end 149.9 55.27269) (width 0.2) (layer "B.Cu") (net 7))
 (segment (start 138.14844 41.86175) (end 139.02906 41.86175) (width 0.2) (layer "B.Cu") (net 7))
 (segment (start 137.52575 42.48444) (end 138.14844 41.86175) (width 0.2) (layer "B.Cu") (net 7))
 (segment (start 138.14844 44.40175) (end 137.52575 43.77906) (width 0.2) (layer "B.Cu") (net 7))
 (segment (start 140.49375 40.39706) (end 140.49375 40.16375) (width 0.2) (layer "B.Cu") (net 7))
 (segment (start 149.9 55.27269) (end 139.02906 44.40175) (width 0.2) (layer "B.Cu") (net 7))
 (segment (start 139.02906 41.86175) (end 140.49375 40.39706) (width 0.2) (layer "B.Cu") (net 7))
 (segment (start 137.52575 43.77906) (end 137.52575 42.48444) (width 0.2) (layer "B.Cu") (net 7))
 (segment (start 139.02906 44.40175) (end 138.14844 44.40175) (width 0.2) (layer "B.Cu") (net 7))
 (segment (start 140.49375 40.16375) (end 138.58875 38.25875) (width 0.2) (layer "B.Cu") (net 7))
 (segment (start 128.30975 67.826) (end 130.17551 67.826) (width 0.2) (layer "F.Cu") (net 14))
 (segment (start 130.84975 53.37975) (end 123.34875 45.87875) (width 0.2) (layer "F.Cu") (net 14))
 (segment (start 130.84975 67.15176) (end 130.84975 53.37975) (width 0.2) (layer "F.Cu") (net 14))
 (segment (start 130.17551 67.826) (end 130.84975 67.15176) (width 0.2) (layer "F.Cu") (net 14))
 (segment (start 127.15875 66.675) (end 128.30975 67.826) (width 0.2) (layer "F.Cu") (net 14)))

